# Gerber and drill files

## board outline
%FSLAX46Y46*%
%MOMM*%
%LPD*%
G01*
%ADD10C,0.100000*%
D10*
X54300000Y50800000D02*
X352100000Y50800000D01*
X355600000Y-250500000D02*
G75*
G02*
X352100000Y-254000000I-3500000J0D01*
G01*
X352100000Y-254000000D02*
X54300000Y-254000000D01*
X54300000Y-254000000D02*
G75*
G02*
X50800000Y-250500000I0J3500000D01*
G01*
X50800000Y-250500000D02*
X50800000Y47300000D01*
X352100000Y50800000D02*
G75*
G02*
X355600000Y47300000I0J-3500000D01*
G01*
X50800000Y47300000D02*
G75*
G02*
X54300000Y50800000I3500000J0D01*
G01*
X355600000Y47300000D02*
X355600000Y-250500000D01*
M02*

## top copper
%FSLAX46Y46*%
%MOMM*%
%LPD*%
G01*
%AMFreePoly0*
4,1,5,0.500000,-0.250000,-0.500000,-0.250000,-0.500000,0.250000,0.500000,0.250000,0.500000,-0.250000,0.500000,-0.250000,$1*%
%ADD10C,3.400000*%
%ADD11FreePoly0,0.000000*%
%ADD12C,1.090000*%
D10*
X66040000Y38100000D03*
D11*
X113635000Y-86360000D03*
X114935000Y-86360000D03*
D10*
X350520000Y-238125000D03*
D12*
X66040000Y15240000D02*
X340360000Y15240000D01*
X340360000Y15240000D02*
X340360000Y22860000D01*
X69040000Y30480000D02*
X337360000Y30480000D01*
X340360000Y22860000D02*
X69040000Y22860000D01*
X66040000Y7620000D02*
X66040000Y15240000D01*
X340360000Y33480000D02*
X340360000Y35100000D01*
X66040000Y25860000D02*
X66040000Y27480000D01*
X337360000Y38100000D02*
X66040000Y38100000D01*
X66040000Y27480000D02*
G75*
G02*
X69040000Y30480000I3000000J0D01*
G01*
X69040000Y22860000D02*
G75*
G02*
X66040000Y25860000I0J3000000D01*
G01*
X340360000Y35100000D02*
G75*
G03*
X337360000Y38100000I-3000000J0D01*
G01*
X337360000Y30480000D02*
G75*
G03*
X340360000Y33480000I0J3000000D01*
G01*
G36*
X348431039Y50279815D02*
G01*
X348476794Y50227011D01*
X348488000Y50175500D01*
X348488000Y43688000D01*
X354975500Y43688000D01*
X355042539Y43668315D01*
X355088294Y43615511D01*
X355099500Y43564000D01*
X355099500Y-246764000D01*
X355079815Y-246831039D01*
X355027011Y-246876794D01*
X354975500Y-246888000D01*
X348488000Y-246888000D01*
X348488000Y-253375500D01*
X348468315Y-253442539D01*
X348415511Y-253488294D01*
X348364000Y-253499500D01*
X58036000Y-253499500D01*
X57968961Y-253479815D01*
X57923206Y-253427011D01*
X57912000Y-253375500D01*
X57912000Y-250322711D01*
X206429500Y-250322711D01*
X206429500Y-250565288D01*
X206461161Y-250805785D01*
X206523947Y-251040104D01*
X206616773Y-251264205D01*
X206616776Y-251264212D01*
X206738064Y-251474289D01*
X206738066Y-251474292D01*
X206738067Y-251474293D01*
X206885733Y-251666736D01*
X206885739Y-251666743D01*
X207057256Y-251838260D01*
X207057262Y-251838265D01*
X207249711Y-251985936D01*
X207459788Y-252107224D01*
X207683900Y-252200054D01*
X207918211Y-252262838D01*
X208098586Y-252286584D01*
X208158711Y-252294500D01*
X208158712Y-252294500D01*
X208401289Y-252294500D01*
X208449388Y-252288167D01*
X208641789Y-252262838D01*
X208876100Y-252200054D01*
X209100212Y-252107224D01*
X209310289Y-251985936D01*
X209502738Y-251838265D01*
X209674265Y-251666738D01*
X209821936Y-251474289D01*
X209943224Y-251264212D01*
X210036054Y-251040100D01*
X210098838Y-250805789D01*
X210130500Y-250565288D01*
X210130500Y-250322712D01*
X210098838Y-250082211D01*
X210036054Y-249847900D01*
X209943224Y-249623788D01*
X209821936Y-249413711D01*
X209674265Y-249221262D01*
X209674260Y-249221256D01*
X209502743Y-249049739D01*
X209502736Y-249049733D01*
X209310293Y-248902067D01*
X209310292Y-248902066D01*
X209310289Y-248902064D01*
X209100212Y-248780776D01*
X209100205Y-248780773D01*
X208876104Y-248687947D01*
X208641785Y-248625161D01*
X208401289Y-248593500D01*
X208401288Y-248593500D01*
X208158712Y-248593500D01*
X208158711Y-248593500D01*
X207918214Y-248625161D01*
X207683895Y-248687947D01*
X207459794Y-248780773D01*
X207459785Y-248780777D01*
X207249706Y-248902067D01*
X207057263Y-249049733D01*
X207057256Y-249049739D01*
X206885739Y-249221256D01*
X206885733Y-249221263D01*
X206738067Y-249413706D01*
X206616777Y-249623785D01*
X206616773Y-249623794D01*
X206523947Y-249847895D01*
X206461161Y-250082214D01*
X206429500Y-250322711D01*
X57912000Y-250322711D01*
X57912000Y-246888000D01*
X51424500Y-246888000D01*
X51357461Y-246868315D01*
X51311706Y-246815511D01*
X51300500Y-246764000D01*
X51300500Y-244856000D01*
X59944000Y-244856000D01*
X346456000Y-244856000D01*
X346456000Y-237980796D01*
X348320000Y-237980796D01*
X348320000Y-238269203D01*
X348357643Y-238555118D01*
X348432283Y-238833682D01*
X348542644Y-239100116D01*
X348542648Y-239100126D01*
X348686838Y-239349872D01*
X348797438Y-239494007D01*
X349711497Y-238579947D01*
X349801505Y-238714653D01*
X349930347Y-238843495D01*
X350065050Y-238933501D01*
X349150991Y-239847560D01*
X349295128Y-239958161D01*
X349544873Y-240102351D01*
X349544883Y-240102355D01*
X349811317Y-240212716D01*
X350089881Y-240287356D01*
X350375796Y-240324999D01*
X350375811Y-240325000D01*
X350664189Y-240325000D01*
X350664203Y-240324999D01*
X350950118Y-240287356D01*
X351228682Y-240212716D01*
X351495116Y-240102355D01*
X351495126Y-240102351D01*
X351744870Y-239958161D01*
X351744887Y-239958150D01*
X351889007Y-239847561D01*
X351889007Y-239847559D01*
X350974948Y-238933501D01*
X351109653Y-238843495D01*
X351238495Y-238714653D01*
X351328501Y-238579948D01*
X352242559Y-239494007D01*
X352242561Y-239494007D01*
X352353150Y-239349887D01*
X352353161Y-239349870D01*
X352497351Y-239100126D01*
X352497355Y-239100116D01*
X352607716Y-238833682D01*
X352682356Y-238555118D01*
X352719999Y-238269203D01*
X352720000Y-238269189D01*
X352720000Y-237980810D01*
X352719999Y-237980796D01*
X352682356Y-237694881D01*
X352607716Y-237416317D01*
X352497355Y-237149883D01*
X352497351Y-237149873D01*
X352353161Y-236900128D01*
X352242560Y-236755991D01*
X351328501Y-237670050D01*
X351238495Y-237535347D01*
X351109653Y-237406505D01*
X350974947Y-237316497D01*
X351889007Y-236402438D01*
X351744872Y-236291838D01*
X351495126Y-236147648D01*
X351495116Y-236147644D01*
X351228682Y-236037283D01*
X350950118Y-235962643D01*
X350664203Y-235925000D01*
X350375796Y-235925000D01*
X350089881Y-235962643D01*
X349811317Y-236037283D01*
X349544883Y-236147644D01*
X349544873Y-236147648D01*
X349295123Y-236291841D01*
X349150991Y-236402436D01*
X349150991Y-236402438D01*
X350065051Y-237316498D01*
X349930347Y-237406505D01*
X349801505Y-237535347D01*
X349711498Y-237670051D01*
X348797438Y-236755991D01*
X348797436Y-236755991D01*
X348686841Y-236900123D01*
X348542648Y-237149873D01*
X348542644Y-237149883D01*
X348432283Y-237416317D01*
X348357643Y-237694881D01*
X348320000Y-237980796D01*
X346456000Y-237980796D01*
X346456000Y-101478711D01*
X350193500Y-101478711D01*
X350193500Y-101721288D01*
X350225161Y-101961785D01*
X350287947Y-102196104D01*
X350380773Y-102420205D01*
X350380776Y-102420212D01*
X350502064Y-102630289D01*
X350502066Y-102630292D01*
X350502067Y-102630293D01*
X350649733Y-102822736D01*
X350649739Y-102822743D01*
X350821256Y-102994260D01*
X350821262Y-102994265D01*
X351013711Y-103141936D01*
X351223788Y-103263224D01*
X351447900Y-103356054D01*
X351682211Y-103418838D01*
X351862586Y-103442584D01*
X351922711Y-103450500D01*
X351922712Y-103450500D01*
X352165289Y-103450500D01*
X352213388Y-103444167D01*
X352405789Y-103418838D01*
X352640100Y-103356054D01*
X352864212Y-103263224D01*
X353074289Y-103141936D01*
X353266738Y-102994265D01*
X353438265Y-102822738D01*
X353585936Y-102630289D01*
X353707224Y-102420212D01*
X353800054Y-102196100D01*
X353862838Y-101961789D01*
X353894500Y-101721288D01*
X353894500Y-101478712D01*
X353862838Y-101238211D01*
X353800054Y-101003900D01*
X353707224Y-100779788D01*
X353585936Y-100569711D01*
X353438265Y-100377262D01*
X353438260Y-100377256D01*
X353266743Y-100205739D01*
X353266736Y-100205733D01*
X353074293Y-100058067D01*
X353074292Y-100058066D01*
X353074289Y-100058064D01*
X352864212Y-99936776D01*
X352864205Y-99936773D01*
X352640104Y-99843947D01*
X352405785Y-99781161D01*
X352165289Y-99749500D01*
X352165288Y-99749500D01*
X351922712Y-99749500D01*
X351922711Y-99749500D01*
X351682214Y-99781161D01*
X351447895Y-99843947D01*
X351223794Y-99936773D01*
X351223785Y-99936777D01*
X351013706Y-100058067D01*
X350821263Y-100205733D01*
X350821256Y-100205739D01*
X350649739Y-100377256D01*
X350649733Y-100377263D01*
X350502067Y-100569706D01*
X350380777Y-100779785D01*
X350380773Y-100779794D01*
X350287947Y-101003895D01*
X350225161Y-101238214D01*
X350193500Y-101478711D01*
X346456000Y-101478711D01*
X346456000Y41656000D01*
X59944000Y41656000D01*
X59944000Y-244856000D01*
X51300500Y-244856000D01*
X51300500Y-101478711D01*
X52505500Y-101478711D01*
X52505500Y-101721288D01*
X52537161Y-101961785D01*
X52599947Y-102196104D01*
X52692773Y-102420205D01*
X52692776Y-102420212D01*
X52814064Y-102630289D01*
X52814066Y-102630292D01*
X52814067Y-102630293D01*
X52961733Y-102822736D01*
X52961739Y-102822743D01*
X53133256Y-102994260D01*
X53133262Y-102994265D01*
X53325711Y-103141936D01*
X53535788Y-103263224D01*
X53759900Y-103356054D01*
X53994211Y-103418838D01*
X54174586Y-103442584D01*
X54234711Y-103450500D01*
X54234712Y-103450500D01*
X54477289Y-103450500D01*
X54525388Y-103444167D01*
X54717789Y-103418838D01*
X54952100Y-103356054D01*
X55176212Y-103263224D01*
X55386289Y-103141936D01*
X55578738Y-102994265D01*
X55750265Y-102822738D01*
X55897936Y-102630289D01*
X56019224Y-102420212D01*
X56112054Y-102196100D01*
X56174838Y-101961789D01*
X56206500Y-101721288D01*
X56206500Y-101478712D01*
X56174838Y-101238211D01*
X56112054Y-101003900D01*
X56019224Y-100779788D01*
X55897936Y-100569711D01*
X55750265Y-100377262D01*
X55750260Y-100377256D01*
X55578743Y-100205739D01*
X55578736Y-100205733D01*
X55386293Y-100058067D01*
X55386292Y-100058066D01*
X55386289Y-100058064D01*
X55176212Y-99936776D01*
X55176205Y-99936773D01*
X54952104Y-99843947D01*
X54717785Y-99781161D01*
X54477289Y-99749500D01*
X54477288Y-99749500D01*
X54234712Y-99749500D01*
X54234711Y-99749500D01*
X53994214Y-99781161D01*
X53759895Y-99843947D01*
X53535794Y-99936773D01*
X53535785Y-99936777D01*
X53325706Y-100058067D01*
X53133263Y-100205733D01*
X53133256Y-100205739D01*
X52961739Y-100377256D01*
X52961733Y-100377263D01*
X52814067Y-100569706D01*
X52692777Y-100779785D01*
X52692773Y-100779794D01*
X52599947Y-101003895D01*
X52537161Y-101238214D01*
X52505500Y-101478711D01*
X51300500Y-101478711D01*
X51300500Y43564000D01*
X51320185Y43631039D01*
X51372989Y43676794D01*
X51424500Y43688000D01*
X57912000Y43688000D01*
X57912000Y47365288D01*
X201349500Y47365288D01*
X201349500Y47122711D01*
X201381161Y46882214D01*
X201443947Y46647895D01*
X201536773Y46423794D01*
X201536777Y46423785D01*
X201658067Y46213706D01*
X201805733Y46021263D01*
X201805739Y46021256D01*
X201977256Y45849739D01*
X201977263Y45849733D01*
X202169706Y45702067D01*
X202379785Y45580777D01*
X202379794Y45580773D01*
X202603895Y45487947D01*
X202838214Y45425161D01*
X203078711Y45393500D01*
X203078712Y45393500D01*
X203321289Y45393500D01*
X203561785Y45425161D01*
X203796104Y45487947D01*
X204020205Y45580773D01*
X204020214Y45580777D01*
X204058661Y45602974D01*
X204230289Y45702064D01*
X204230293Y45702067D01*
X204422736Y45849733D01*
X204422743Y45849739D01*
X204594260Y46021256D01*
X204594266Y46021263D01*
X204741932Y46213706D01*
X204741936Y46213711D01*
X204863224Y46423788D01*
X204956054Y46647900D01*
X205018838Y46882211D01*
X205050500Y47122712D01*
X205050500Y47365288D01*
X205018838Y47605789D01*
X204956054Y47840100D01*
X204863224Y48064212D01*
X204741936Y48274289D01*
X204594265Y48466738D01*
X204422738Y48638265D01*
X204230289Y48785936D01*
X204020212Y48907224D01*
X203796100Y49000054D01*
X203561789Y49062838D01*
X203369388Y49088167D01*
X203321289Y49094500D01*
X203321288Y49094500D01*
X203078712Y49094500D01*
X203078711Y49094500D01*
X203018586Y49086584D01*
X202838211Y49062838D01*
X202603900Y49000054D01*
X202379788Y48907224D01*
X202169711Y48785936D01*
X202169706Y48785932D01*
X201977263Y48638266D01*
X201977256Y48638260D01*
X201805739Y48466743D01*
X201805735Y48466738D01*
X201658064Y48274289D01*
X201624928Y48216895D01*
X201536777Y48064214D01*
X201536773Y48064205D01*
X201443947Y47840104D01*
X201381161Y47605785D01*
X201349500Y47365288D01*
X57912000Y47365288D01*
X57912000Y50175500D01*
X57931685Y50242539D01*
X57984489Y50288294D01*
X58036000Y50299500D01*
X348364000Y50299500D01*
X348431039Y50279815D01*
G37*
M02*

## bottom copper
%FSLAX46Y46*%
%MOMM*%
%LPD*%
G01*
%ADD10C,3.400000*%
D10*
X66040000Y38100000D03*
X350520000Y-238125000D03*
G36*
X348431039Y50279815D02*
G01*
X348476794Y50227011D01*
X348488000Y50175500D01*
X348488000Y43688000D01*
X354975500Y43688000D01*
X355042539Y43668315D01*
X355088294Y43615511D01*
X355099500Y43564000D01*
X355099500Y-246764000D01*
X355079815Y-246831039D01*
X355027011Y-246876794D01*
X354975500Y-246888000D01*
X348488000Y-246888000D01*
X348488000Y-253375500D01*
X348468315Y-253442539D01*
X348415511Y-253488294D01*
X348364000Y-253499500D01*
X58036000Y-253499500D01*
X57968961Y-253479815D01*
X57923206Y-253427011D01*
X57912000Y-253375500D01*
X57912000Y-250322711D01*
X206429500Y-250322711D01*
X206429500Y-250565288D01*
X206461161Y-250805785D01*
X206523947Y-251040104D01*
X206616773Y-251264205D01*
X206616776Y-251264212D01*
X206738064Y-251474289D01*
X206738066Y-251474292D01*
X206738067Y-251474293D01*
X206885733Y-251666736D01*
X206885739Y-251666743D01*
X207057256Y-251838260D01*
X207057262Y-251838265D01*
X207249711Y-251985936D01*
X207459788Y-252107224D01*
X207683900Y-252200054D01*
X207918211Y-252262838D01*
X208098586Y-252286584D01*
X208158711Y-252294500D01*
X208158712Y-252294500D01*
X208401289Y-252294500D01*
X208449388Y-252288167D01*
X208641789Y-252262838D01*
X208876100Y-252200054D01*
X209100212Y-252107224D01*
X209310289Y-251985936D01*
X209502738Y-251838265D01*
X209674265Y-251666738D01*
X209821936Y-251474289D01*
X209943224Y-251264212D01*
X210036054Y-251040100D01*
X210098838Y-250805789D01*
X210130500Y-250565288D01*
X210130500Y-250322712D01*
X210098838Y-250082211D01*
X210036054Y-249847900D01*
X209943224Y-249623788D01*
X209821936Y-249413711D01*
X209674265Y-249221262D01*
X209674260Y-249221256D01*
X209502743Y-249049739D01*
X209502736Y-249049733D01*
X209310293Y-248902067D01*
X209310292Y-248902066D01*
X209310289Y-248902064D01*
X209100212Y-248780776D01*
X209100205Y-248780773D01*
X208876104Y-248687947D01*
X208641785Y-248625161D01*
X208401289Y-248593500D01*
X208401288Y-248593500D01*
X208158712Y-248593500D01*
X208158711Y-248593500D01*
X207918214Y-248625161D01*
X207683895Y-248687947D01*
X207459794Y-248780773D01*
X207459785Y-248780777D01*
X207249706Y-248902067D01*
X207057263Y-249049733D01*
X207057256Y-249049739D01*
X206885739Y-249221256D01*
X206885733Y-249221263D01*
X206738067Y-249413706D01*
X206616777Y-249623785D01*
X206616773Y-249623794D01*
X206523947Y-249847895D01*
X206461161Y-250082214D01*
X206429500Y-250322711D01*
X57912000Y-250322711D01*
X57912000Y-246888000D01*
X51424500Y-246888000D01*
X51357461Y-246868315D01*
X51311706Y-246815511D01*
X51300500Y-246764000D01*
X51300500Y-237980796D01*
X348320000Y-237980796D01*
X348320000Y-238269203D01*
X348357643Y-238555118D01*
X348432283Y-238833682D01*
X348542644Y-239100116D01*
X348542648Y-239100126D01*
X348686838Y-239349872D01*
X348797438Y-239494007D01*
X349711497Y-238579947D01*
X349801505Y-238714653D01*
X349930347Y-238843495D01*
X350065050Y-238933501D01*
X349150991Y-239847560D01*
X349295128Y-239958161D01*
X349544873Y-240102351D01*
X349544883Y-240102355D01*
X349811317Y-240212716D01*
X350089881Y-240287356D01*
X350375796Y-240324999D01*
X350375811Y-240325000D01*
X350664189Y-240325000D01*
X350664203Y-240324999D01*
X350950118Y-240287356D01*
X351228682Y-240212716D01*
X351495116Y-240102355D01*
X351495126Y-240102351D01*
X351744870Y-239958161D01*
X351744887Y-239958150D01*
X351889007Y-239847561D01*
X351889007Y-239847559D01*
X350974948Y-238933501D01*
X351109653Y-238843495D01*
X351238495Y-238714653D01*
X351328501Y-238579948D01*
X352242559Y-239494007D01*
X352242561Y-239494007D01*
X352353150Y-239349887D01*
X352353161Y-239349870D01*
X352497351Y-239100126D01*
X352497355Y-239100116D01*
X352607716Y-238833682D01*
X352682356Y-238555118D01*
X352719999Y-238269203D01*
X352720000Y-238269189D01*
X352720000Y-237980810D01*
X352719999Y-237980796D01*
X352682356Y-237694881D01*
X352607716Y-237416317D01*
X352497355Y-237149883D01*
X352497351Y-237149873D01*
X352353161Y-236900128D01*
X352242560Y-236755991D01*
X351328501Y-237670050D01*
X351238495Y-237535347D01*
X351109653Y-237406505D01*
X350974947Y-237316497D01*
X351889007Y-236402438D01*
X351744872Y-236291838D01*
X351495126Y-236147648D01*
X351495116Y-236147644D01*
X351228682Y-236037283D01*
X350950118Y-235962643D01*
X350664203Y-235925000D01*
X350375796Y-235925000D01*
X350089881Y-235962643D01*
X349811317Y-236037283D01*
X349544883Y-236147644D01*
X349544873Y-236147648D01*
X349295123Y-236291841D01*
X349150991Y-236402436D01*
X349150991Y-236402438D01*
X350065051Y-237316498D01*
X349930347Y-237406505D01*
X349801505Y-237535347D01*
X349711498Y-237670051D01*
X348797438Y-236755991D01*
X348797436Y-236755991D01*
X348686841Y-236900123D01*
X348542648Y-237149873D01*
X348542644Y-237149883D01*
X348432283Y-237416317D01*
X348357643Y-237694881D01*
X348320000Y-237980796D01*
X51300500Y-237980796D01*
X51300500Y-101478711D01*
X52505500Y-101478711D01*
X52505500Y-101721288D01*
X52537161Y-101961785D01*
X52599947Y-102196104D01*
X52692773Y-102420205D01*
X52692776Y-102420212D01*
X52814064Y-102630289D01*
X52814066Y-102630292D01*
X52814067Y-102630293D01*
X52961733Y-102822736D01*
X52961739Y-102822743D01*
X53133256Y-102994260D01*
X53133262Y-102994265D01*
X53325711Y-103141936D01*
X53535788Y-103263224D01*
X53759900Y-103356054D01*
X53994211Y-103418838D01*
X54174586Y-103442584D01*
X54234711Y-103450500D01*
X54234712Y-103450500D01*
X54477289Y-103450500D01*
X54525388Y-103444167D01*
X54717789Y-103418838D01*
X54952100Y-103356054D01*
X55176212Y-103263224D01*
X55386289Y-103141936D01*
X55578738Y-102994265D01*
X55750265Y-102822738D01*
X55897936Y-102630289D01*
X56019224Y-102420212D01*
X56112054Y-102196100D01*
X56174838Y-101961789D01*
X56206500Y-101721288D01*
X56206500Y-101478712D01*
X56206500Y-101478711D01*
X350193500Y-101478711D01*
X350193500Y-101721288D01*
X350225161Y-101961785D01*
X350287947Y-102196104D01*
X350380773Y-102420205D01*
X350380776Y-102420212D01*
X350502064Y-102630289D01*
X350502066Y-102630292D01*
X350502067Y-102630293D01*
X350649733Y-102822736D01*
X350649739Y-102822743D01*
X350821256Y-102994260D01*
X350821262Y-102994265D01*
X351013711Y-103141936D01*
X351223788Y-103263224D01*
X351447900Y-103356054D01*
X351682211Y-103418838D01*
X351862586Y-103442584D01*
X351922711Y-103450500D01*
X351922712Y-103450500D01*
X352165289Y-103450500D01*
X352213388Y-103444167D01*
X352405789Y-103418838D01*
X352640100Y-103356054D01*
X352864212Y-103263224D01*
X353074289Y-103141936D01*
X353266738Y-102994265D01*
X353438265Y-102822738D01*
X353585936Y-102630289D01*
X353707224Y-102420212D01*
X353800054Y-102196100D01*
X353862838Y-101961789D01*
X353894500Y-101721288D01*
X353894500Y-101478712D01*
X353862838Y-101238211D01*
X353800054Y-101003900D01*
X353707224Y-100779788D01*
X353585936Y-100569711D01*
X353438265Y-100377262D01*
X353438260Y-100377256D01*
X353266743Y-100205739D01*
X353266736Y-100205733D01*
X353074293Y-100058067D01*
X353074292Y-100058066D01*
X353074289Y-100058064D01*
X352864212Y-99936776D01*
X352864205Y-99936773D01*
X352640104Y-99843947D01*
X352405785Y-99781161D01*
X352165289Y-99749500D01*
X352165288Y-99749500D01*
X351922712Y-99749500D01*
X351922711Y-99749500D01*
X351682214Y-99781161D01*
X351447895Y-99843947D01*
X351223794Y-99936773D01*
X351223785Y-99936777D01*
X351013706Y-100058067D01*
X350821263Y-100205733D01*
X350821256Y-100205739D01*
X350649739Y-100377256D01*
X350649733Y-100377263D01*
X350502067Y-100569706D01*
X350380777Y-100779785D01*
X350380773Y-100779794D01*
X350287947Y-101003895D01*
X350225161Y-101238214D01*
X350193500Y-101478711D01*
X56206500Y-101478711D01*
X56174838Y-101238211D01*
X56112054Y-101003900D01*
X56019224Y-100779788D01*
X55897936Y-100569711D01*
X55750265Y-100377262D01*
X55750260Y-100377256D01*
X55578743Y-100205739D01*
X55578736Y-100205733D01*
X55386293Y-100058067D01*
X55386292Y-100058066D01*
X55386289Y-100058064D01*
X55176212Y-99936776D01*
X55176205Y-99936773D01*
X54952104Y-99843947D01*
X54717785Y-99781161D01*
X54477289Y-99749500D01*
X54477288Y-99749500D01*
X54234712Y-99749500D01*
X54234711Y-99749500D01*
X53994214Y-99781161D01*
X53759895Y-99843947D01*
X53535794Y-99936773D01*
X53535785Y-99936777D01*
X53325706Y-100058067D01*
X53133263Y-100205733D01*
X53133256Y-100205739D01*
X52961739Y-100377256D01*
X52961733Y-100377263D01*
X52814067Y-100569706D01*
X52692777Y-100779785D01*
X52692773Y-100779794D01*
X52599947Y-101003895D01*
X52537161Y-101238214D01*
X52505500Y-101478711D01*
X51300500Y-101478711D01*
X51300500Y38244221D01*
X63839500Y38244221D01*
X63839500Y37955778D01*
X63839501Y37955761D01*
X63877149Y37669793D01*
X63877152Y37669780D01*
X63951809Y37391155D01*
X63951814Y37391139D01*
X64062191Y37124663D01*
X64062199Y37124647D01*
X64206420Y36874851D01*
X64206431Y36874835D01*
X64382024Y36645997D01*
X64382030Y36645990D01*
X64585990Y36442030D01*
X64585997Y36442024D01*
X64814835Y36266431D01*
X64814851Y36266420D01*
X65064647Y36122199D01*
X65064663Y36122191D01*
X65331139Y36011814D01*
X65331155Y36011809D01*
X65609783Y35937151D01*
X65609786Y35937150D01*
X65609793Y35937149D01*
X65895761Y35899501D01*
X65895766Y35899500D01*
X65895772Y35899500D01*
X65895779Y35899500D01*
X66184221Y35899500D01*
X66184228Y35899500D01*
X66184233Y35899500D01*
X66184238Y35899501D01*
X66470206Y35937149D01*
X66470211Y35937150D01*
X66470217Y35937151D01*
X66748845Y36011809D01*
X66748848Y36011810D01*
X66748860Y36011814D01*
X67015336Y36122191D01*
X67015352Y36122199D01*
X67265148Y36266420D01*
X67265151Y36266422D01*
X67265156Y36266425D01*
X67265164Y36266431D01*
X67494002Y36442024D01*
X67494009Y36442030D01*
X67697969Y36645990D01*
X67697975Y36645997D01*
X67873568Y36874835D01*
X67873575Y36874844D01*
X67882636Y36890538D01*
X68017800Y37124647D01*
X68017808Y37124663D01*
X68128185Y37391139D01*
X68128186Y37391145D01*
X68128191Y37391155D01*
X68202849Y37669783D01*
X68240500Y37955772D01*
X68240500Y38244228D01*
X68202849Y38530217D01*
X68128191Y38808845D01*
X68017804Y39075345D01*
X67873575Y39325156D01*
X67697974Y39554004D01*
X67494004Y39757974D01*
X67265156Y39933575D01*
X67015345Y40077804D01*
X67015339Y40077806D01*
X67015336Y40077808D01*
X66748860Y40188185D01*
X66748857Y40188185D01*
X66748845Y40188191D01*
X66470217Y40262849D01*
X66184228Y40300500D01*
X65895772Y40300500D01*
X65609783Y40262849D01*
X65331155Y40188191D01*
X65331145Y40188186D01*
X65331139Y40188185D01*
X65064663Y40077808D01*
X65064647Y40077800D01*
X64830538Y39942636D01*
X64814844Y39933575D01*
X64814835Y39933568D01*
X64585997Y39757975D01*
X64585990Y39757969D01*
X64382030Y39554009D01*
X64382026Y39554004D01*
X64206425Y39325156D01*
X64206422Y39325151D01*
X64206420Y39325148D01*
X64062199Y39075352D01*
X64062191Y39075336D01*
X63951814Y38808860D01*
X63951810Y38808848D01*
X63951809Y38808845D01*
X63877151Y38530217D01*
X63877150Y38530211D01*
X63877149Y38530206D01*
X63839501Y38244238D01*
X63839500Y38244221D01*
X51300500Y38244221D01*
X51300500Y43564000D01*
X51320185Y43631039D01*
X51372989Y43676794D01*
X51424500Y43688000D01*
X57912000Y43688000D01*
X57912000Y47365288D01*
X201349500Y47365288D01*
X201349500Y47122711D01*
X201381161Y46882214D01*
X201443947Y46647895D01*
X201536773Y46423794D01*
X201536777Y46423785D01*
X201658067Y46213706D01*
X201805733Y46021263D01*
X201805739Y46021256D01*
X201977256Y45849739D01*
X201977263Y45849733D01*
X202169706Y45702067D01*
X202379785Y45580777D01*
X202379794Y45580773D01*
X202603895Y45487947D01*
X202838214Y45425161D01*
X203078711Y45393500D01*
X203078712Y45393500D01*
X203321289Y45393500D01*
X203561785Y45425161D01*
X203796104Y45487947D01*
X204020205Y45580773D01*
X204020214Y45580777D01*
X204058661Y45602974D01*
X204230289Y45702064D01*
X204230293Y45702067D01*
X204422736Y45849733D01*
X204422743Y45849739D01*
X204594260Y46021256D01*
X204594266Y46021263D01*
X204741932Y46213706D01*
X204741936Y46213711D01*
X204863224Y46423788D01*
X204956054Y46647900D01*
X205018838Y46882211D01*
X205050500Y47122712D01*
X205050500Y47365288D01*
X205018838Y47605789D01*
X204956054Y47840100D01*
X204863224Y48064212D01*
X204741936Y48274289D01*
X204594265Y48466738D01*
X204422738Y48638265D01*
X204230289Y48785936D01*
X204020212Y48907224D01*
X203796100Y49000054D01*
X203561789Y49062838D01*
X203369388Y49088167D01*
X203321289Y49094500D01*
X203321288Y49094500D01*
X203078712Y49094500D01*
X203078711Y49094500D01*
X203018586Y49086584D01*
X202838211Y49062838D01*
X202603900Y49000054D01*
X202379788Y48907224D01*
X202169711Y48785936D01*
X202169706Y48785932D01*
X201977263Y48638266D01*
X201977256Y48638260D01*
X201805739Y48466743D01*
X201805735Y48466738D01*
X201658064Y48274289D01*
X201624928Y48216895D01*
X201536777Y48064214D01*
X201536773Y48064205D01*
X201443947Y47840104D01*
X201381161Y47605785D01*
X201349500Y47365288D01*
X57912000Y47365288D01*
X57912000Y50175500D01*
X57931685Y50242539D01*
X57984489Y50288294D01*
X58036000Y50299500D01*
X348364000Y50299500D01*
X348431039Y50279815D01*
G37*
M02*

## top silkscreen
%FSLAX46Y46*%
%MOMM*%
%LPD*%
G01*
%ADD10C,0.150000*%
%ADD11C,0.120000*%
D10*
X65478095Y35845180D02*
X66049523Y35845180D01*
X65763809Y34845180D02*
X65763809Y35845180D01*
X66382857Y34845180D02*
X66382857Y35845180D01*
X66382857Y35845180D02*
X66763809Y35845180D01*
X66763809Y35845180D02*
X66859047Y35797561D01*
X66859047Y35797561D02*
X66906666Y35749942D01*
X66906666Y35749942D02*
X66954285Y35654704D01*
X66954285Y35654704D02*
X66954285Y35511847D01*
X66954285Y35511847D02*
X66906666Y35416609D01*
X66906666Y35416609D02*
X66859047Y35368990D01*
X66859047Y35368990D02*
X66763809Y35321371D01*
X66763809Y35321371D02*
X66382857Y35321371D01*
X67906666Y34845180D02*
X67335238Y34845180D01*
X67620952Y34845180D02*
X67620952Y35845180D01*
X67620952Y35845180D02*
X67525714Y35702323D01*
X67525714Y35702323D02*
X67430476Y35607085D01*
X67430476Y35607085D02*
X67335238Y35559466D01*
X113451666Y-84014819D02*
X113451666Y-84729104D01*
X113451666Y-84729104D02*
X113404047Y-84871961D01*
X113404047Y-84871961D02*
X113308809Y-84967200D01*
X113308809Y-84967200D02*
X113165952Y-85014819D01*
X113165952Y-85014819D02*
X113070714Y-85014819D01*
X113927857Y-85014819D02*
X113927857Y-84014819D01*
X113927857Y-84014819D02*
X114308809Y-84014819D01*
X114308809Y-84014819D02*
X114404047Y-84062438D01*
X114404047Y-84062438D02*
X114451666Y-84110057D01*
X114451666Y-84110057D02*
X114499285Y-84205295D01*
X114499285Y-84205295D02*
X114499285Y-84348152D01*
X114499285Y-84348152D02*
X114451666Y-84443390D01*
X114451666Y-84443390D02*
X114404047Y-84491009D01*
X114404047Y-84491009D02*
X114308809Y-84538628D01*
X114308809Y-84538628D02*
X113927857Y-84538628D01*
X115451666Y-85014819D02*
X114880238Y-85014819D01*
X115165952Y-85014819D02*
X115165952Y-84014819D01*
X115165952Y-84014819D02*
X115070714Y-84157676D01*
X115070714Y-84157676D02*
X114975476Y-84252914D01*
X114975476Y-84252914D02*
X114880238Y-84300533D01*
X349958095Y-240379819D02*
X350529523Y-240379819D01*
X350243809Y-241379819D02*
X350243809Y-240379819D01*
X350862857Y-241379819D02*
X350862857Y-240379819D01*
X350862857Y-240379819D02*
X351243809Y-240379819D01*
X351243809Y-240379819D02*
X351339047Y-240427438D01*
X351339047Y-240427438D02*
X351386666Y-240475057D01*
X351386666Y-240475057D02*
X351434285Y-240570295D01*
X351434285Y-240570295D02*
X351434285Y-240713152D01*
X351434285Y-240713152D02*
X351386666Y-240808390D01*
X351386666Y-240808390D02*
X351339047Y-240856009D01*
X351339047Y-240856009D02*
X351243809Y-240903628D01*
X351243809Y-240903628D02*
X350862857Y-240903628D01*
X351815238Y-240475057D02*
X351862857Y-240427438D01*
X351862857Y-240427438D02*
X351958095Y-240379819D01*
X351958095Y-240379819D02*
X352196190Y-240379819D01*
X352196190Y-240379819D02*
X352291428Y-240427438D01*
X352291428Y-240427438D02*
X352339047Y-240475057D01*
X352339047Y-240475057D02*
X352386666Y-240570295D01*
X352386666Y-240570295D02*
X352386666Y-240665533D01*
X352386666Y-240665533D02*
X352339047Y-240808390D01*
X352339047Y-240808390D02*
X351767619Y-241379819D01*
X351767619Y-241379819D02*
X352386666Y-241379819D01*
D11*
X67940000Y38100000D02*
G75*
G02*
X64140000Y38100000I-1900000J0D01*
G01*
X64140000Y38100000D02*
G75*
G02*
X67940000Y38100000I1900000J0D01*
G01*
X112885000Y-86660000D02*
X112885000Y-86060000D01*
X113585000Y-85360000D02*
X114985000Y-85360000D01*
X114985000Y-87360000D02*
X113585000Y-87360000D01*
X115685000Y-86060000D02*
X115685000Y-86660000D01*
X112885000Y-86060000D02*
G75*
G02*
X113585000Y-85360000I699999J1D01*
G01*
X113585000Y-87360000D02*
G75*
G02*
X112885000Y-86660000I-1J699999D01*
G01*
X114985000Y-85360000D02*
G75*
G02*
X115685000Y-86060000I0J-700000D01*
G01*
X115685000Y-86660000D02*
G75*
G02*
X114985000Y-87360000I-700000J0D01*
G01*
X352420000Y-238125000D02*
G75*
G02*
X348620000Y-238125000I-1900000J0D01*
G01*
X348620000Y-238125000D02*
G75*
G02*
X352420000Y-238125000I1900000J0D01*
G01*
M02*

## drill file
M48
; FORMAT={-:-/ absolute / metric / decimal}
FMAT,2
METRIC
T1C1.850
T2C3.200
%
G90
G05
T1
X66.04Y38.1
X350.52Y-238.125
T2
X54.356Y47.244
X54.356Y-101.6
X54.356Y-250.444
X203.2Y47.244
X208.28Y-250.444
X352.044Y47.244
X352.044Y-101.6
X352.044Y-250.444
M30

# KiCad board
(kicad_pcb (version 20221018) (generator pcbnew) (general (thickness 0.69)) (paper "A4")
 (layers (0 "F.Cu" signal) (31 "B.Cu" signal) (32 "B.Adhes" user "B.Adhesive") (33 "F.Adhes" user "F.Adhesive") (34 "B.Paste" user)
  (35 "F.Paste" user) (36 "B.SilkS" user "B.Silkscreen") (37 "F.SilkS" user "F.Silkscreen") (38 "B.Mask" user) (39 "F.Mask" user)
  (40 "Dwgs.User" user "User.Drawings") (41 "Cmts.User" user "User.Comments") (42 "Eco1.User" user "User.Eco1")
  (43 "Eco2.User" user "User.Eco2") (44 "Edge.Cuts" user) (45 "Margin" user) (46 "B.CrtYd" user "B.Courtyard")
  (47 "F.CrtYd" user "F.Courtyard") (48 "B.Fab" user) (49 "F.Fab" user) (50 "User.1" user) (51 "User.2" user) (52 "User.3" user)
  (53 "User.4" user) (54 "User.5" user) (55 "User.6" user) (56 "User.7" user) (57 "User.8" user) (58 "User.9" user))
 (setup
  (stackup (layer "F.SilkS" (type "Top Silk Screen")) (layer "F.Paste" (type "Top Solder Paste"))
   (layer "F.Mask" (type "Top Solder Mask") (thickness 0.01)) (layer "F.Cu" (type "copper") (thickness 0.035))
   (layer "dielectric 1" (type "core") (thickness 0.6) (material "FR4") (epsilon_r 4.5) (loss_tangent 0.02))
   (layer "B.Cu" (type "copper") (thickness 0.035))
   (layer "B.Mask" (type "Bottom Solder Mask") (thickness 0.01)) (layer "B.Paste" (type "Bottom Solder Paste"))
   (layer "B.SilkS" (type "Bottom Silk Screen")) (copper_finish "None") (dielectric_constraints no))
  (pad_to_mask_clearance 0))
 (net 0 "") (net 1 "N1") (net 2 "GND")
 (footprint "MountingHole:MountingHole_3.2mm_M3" (layer "F.Cu") (at 203.2 -47.244)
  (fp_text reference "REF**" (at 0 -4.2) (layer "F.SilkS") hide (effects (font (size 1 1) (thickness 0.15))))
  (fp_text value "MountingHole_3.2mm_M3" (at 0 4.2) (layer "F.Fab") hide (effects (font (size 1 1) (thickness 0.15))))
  (pad "" np_thru_hole circle (at 0 0) (size 3.2 3.2) (drill 3.2) (layers "F&B.Cu" "*.Mask")))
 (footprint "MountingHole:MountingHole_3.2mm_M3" (layer "F.Cu") (at 208.28 250.444)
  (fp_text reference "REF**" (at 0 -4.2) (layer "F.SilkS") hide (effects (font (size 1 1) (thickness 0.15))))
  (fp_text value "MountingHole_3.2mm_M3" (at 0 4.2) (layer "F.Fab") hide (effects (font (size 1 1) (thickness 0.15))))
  (pad "" np_thru_hole circle (at 0 0) (size 3.2 3.2) (drill 3.2) (layers "F&B.Cu" "*.Mask")))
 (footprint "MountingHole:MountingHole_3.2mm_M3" (layer "F.Cu") (at 54.356 101.6)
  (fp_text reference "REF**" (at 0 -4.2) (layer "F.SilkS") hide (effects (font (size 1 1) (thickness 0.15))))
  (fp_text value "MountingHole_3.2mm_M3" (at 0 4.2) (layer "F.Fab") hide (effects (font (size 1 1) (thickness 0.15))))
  (pad "" np_thru_hole circle (at 0 0) (size 3.2 3.2) (drill 3.2) (layers "F&B.Cu" "*.Mask")))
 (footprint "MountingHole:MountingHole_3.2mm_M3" (layer "F.Cu") (at 352.044 250.444)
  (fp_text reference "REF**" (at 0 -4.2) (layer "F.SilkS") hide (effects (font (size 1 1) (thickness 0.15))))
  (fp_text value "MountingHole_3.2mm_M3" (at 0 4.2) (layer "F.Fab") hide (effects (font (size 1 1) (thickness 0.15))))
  (pad "" np_thru_hole circle (at 0 0) (size 3.2 3.2) (drill 3.2) (layers "F&B.Cu" "*.Mask")))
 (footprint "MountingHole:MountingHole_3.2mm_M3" (layer "F.Cu") (at 54.356 250.444)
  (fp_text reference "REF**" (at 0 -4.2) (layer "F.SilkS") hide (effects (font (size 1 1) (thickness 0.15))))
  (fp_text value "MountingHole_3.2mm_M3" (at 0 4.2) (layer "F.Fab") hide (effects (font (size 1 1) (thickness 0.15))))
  (pad "" np_thru_hole circle (at 0 0) (size 3.2 3.2) (drill 3.2) (layers "F&B.Cu" "*.Mask")))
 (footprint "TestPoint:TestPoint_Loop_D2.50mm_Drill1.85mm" (layer "F.Cu") (at 66.04 -38.1)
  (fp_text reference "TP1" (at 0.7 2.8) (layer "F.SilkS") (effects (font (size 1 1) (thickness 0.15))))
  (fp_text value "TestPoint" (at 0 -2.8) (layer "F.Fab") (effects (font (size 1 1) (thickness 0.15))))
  (fp_circle (center 0 0) (end 1.9 0) (stroke (width 0.12) (type solid)) (fill none) (layer "F.SilkS"))
  (pad "1" thru_hole circle (at 0 0) (size 3.4 3.4) (drill 1.85) (layers "*.Cu" "*.Mask") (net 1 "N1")))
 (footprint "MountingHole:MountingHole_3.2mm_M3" (layer "F.Cu") (at 352.044 -47.244)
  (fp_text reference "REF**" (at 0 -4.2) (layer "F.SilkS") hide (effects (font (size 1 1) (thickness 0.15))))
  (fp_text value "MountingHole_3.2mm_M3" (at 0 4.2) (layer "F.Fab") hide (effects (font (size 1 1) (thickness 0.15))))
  (pad "" np_thru_hole circle (at 0 0) (size 3.2 3.2) (drill 3.2) (layers "F&B.Cu" "*.Mask")))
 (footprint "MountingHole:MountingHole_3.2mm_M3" (layer "F.Cu") (at 54.356 -47.244)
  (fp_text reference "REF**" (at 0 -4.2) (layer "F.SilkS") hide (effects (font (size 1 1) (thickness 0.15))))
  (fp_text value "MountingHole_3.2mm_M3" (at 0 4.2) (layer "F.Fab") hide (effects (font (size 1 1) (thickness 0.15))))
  (pad "" np_thru_hole circle (at 0 0) (size 3.2 3.2) (drill 3.2) (layers "*.Cu" "*.Mask")))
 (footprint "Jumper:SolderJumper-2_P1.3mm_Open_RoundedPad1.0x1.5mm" (layer "F.Cu") (at 114.285 86.36)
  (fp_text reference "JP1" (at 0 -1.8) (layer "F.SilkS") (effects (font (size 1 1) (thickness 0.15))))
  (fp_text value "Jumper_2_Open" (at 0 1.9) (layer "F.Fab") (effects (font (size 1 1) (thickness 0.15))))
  (fp_line (start -1.4 0.3) (end -1.4 -0.3) (stroke (width 0.12) (type solid)) (layer "F.SilkS"))
  (fp_line (start -0.7 -1) (end 0.7 -1) (stroke (width 0.12) (type solid)) (layer "F.SilkS"))
  (fp_line (start 0.7 1) (end -0.7 1) (stroke (width 0.12) (type solid)) (layer "F.SilkS"))
  (fp_line (start 1.4 -0.3) (end 1.4 0.3) (stroke (width 0.12) (type solid)) (layer "F.SilkS"))
  (fp_arc (start -1.4 -0.3) (mid -1.194975 -0.794975) (end -0.7 -1) (stroke (width 0.12) (type solid)) (layer "F.SilkS"))
  (fp_arc (start -0.7 1) (mid -1.194975 0.794975) (end -1.4 0.3) (stroke (width 0.12) (type solid)) (layer "F.SilkS"))
  (fp_arc (start 0.7 -1) (mid 1.194975 -0.794975) (end 1.4 -0.3) (stroke (width 0.12) (type solid)) (layer "F.SilkS"))
  (fp_arc (start 1.4 0.3) (mid 1.194975 0.794975) (end 0.7 1) (stroke (width 0.12) (type solid)) (layer "F.SilkS"))
  (pad "1" smd custom (at -0.65 0) (size 1 0.5) (layers "F.Cu" "F.Mask") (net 1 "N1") (zone_connect 2) (thermal_bridge_angle 45)
   (options (clearance outline) (anchor rect)) (primitives))
  (pad "2" smd custom (at 0.65 0) (size 1 0.5) (layers "F.Cu" "F.Mask") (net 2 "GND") (zone_connect 2) (thermal_bridge_angle 45)
   (options (clearance outline) (anchor rect)) (primitives)))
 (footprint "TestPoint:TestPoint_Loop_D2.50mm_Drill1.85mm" (layer "F.Cu") (at 350.52 238.125)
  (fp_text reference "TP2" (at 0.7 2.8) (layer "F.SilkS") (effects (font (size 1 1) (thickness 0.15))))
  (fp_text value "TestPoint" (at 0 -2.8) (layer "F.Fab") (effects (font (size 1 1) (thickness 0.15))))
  (fp_circle (center 0 0) (end 1.9 0) (stroke (width 0.12) (type solid)) (fill none) (layer "F.SilkS"))
  (pad "1" thru_hole circle (at 0 0) (size 3.4 3.4) (drill 1.85) (layers "*.Cu" "*.Mask") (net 2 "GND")))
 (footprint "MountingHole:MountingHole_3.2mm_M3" (layer "F.Cu") (at 352.044 101.6)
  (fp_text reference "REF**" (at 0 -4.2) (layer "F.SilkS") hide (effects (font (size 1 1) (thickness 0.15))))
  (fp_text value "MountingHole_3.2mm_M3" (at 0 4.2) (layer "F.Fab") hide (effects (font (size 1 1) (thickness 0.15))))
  (pad "" np_thru_hole circle (at 0 0) (size 3.2 3.2) (drill 3.2) (layers "F&B.Cu" "*.Mask")))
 (gr_line (start 54.3 -50.8) (end 352.1 -50.8) (stroke (width 0.1) (type default)) (layer "Edge.Cuts"))
 (gr_arc (start 355.6 250.5) (mid 354.574874 252.974874) (end 352.1 254) (stroke (width 0.1) (type default)) (layer "Edge.Cuts"))
 (gr_line (start 352.1 254) (end 54.3 254) (stroke (width 0.1) (type default)) (layer "Edge.Cuts"))
 (gr_arc (start 54.3 254) (mid 51.825126 252.974874) (end 50.8 250.5) (stroke (width 0.1) (type default)) (layer "Edge.Cuts"))
 (gr_line (start 50.8 250.5) (end 50.8 -47.3) (stroke (width 0.1) (type default)) (layer "Edge.Cuts"))
 (gr_arc (start 352.1 -50.8) (mid 354.574874 -49.774874) (end 355.6 -47.3) (stroke (width 0.1) (type default)) (layer "Edge.Cuts"))
 (gr_arc (start 50.8 -47.3) (mid 51.825126 -49.774874) (end 54.3 -50.8) (stroke (width 0.1) (type default)) (layer "Edge.Cuts"))
 (gr_line (start 355.6 -47.3) (end 355.6 250.5) (stroke (width 0.1) (type default)) (layer "Edge.Cuts"))
 (segment (start 66.04 -15.24) (end 340.36 -15.24) (width 1.09) (layer "F.Cu") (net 1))
 (segment (start 340.36 -15.24) (end 340.36 -22.86) (width 1.09) (layer "F.Cu") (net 1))
 (segment (start 69.04 -30.48) (end 337.36 -30.48) (width 1.09) (layer "F.Cu") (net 1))
 (segment (start 340.36 -22.86) (end 69.04 -22.86) (width 1.09) (layer "F.Cu") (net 1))
 (segment (start 66.04 -7.62) (end 66.04 -15.24) (width 1.09) (layer "F.Cu") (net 1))
 (segment (start 340.36 -33.48) (end 340.36 -35.1) (width 1.09) (layer "F.Cu") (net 1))
 (segment (start 66.04 -25.86) (end 66.04 -27.48) (width 1.09) (layer "F.Cu") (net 1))
 (segment (start 337.36 -38.1) (end 66.04 -38.1) (width 1.09) (layer "F.Cu") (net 1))
 (arc (start 66.04 -27.48) (mid 66.91868 -29.60132) (end 69.04 -30.48) (width 1.09) (layer "F.Cu") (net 1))
 (arc (start 69.04 -22.86) (mid 66.91868 -23.73868) (end 66.04 -25.86) (width 1.09) (layer "F.Cu") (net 1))
 (arc (start 340.36 -35.1) (mid 339.48132 -37.22132) (end 337.36 -38.1) (width 1.09) (layer "F.Cu") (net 1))
 (arc (start 337.36 -30.48) (mid 339.48132 -31.35868) (end 340.36 -33.48) (width 1.09) (layer "F.Cu") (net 1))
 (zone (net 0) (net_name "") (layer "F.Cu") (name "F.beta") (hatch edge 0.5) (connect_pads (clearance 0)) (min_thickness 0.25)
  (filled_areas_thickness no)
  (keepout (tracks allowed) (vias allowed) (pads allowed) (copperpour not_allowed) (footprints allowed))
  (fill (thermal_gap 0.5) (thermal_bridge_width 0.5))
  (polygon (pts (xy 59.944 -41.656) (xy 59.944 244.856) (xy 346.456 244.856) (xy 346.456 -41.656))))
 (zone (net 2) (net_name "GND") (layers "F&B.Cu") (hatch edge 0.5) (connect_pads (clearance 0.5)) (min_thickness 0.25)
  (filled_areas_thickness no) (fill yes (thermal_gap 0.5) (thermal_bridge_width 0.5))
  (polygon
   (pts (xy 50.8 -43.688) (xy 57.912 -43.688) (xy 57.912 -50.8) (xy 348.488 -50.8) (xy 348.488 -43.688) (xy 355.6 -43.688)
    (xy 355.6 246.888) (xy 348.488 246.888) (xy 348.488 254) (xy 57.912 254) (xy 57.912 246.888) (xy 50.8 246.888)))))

